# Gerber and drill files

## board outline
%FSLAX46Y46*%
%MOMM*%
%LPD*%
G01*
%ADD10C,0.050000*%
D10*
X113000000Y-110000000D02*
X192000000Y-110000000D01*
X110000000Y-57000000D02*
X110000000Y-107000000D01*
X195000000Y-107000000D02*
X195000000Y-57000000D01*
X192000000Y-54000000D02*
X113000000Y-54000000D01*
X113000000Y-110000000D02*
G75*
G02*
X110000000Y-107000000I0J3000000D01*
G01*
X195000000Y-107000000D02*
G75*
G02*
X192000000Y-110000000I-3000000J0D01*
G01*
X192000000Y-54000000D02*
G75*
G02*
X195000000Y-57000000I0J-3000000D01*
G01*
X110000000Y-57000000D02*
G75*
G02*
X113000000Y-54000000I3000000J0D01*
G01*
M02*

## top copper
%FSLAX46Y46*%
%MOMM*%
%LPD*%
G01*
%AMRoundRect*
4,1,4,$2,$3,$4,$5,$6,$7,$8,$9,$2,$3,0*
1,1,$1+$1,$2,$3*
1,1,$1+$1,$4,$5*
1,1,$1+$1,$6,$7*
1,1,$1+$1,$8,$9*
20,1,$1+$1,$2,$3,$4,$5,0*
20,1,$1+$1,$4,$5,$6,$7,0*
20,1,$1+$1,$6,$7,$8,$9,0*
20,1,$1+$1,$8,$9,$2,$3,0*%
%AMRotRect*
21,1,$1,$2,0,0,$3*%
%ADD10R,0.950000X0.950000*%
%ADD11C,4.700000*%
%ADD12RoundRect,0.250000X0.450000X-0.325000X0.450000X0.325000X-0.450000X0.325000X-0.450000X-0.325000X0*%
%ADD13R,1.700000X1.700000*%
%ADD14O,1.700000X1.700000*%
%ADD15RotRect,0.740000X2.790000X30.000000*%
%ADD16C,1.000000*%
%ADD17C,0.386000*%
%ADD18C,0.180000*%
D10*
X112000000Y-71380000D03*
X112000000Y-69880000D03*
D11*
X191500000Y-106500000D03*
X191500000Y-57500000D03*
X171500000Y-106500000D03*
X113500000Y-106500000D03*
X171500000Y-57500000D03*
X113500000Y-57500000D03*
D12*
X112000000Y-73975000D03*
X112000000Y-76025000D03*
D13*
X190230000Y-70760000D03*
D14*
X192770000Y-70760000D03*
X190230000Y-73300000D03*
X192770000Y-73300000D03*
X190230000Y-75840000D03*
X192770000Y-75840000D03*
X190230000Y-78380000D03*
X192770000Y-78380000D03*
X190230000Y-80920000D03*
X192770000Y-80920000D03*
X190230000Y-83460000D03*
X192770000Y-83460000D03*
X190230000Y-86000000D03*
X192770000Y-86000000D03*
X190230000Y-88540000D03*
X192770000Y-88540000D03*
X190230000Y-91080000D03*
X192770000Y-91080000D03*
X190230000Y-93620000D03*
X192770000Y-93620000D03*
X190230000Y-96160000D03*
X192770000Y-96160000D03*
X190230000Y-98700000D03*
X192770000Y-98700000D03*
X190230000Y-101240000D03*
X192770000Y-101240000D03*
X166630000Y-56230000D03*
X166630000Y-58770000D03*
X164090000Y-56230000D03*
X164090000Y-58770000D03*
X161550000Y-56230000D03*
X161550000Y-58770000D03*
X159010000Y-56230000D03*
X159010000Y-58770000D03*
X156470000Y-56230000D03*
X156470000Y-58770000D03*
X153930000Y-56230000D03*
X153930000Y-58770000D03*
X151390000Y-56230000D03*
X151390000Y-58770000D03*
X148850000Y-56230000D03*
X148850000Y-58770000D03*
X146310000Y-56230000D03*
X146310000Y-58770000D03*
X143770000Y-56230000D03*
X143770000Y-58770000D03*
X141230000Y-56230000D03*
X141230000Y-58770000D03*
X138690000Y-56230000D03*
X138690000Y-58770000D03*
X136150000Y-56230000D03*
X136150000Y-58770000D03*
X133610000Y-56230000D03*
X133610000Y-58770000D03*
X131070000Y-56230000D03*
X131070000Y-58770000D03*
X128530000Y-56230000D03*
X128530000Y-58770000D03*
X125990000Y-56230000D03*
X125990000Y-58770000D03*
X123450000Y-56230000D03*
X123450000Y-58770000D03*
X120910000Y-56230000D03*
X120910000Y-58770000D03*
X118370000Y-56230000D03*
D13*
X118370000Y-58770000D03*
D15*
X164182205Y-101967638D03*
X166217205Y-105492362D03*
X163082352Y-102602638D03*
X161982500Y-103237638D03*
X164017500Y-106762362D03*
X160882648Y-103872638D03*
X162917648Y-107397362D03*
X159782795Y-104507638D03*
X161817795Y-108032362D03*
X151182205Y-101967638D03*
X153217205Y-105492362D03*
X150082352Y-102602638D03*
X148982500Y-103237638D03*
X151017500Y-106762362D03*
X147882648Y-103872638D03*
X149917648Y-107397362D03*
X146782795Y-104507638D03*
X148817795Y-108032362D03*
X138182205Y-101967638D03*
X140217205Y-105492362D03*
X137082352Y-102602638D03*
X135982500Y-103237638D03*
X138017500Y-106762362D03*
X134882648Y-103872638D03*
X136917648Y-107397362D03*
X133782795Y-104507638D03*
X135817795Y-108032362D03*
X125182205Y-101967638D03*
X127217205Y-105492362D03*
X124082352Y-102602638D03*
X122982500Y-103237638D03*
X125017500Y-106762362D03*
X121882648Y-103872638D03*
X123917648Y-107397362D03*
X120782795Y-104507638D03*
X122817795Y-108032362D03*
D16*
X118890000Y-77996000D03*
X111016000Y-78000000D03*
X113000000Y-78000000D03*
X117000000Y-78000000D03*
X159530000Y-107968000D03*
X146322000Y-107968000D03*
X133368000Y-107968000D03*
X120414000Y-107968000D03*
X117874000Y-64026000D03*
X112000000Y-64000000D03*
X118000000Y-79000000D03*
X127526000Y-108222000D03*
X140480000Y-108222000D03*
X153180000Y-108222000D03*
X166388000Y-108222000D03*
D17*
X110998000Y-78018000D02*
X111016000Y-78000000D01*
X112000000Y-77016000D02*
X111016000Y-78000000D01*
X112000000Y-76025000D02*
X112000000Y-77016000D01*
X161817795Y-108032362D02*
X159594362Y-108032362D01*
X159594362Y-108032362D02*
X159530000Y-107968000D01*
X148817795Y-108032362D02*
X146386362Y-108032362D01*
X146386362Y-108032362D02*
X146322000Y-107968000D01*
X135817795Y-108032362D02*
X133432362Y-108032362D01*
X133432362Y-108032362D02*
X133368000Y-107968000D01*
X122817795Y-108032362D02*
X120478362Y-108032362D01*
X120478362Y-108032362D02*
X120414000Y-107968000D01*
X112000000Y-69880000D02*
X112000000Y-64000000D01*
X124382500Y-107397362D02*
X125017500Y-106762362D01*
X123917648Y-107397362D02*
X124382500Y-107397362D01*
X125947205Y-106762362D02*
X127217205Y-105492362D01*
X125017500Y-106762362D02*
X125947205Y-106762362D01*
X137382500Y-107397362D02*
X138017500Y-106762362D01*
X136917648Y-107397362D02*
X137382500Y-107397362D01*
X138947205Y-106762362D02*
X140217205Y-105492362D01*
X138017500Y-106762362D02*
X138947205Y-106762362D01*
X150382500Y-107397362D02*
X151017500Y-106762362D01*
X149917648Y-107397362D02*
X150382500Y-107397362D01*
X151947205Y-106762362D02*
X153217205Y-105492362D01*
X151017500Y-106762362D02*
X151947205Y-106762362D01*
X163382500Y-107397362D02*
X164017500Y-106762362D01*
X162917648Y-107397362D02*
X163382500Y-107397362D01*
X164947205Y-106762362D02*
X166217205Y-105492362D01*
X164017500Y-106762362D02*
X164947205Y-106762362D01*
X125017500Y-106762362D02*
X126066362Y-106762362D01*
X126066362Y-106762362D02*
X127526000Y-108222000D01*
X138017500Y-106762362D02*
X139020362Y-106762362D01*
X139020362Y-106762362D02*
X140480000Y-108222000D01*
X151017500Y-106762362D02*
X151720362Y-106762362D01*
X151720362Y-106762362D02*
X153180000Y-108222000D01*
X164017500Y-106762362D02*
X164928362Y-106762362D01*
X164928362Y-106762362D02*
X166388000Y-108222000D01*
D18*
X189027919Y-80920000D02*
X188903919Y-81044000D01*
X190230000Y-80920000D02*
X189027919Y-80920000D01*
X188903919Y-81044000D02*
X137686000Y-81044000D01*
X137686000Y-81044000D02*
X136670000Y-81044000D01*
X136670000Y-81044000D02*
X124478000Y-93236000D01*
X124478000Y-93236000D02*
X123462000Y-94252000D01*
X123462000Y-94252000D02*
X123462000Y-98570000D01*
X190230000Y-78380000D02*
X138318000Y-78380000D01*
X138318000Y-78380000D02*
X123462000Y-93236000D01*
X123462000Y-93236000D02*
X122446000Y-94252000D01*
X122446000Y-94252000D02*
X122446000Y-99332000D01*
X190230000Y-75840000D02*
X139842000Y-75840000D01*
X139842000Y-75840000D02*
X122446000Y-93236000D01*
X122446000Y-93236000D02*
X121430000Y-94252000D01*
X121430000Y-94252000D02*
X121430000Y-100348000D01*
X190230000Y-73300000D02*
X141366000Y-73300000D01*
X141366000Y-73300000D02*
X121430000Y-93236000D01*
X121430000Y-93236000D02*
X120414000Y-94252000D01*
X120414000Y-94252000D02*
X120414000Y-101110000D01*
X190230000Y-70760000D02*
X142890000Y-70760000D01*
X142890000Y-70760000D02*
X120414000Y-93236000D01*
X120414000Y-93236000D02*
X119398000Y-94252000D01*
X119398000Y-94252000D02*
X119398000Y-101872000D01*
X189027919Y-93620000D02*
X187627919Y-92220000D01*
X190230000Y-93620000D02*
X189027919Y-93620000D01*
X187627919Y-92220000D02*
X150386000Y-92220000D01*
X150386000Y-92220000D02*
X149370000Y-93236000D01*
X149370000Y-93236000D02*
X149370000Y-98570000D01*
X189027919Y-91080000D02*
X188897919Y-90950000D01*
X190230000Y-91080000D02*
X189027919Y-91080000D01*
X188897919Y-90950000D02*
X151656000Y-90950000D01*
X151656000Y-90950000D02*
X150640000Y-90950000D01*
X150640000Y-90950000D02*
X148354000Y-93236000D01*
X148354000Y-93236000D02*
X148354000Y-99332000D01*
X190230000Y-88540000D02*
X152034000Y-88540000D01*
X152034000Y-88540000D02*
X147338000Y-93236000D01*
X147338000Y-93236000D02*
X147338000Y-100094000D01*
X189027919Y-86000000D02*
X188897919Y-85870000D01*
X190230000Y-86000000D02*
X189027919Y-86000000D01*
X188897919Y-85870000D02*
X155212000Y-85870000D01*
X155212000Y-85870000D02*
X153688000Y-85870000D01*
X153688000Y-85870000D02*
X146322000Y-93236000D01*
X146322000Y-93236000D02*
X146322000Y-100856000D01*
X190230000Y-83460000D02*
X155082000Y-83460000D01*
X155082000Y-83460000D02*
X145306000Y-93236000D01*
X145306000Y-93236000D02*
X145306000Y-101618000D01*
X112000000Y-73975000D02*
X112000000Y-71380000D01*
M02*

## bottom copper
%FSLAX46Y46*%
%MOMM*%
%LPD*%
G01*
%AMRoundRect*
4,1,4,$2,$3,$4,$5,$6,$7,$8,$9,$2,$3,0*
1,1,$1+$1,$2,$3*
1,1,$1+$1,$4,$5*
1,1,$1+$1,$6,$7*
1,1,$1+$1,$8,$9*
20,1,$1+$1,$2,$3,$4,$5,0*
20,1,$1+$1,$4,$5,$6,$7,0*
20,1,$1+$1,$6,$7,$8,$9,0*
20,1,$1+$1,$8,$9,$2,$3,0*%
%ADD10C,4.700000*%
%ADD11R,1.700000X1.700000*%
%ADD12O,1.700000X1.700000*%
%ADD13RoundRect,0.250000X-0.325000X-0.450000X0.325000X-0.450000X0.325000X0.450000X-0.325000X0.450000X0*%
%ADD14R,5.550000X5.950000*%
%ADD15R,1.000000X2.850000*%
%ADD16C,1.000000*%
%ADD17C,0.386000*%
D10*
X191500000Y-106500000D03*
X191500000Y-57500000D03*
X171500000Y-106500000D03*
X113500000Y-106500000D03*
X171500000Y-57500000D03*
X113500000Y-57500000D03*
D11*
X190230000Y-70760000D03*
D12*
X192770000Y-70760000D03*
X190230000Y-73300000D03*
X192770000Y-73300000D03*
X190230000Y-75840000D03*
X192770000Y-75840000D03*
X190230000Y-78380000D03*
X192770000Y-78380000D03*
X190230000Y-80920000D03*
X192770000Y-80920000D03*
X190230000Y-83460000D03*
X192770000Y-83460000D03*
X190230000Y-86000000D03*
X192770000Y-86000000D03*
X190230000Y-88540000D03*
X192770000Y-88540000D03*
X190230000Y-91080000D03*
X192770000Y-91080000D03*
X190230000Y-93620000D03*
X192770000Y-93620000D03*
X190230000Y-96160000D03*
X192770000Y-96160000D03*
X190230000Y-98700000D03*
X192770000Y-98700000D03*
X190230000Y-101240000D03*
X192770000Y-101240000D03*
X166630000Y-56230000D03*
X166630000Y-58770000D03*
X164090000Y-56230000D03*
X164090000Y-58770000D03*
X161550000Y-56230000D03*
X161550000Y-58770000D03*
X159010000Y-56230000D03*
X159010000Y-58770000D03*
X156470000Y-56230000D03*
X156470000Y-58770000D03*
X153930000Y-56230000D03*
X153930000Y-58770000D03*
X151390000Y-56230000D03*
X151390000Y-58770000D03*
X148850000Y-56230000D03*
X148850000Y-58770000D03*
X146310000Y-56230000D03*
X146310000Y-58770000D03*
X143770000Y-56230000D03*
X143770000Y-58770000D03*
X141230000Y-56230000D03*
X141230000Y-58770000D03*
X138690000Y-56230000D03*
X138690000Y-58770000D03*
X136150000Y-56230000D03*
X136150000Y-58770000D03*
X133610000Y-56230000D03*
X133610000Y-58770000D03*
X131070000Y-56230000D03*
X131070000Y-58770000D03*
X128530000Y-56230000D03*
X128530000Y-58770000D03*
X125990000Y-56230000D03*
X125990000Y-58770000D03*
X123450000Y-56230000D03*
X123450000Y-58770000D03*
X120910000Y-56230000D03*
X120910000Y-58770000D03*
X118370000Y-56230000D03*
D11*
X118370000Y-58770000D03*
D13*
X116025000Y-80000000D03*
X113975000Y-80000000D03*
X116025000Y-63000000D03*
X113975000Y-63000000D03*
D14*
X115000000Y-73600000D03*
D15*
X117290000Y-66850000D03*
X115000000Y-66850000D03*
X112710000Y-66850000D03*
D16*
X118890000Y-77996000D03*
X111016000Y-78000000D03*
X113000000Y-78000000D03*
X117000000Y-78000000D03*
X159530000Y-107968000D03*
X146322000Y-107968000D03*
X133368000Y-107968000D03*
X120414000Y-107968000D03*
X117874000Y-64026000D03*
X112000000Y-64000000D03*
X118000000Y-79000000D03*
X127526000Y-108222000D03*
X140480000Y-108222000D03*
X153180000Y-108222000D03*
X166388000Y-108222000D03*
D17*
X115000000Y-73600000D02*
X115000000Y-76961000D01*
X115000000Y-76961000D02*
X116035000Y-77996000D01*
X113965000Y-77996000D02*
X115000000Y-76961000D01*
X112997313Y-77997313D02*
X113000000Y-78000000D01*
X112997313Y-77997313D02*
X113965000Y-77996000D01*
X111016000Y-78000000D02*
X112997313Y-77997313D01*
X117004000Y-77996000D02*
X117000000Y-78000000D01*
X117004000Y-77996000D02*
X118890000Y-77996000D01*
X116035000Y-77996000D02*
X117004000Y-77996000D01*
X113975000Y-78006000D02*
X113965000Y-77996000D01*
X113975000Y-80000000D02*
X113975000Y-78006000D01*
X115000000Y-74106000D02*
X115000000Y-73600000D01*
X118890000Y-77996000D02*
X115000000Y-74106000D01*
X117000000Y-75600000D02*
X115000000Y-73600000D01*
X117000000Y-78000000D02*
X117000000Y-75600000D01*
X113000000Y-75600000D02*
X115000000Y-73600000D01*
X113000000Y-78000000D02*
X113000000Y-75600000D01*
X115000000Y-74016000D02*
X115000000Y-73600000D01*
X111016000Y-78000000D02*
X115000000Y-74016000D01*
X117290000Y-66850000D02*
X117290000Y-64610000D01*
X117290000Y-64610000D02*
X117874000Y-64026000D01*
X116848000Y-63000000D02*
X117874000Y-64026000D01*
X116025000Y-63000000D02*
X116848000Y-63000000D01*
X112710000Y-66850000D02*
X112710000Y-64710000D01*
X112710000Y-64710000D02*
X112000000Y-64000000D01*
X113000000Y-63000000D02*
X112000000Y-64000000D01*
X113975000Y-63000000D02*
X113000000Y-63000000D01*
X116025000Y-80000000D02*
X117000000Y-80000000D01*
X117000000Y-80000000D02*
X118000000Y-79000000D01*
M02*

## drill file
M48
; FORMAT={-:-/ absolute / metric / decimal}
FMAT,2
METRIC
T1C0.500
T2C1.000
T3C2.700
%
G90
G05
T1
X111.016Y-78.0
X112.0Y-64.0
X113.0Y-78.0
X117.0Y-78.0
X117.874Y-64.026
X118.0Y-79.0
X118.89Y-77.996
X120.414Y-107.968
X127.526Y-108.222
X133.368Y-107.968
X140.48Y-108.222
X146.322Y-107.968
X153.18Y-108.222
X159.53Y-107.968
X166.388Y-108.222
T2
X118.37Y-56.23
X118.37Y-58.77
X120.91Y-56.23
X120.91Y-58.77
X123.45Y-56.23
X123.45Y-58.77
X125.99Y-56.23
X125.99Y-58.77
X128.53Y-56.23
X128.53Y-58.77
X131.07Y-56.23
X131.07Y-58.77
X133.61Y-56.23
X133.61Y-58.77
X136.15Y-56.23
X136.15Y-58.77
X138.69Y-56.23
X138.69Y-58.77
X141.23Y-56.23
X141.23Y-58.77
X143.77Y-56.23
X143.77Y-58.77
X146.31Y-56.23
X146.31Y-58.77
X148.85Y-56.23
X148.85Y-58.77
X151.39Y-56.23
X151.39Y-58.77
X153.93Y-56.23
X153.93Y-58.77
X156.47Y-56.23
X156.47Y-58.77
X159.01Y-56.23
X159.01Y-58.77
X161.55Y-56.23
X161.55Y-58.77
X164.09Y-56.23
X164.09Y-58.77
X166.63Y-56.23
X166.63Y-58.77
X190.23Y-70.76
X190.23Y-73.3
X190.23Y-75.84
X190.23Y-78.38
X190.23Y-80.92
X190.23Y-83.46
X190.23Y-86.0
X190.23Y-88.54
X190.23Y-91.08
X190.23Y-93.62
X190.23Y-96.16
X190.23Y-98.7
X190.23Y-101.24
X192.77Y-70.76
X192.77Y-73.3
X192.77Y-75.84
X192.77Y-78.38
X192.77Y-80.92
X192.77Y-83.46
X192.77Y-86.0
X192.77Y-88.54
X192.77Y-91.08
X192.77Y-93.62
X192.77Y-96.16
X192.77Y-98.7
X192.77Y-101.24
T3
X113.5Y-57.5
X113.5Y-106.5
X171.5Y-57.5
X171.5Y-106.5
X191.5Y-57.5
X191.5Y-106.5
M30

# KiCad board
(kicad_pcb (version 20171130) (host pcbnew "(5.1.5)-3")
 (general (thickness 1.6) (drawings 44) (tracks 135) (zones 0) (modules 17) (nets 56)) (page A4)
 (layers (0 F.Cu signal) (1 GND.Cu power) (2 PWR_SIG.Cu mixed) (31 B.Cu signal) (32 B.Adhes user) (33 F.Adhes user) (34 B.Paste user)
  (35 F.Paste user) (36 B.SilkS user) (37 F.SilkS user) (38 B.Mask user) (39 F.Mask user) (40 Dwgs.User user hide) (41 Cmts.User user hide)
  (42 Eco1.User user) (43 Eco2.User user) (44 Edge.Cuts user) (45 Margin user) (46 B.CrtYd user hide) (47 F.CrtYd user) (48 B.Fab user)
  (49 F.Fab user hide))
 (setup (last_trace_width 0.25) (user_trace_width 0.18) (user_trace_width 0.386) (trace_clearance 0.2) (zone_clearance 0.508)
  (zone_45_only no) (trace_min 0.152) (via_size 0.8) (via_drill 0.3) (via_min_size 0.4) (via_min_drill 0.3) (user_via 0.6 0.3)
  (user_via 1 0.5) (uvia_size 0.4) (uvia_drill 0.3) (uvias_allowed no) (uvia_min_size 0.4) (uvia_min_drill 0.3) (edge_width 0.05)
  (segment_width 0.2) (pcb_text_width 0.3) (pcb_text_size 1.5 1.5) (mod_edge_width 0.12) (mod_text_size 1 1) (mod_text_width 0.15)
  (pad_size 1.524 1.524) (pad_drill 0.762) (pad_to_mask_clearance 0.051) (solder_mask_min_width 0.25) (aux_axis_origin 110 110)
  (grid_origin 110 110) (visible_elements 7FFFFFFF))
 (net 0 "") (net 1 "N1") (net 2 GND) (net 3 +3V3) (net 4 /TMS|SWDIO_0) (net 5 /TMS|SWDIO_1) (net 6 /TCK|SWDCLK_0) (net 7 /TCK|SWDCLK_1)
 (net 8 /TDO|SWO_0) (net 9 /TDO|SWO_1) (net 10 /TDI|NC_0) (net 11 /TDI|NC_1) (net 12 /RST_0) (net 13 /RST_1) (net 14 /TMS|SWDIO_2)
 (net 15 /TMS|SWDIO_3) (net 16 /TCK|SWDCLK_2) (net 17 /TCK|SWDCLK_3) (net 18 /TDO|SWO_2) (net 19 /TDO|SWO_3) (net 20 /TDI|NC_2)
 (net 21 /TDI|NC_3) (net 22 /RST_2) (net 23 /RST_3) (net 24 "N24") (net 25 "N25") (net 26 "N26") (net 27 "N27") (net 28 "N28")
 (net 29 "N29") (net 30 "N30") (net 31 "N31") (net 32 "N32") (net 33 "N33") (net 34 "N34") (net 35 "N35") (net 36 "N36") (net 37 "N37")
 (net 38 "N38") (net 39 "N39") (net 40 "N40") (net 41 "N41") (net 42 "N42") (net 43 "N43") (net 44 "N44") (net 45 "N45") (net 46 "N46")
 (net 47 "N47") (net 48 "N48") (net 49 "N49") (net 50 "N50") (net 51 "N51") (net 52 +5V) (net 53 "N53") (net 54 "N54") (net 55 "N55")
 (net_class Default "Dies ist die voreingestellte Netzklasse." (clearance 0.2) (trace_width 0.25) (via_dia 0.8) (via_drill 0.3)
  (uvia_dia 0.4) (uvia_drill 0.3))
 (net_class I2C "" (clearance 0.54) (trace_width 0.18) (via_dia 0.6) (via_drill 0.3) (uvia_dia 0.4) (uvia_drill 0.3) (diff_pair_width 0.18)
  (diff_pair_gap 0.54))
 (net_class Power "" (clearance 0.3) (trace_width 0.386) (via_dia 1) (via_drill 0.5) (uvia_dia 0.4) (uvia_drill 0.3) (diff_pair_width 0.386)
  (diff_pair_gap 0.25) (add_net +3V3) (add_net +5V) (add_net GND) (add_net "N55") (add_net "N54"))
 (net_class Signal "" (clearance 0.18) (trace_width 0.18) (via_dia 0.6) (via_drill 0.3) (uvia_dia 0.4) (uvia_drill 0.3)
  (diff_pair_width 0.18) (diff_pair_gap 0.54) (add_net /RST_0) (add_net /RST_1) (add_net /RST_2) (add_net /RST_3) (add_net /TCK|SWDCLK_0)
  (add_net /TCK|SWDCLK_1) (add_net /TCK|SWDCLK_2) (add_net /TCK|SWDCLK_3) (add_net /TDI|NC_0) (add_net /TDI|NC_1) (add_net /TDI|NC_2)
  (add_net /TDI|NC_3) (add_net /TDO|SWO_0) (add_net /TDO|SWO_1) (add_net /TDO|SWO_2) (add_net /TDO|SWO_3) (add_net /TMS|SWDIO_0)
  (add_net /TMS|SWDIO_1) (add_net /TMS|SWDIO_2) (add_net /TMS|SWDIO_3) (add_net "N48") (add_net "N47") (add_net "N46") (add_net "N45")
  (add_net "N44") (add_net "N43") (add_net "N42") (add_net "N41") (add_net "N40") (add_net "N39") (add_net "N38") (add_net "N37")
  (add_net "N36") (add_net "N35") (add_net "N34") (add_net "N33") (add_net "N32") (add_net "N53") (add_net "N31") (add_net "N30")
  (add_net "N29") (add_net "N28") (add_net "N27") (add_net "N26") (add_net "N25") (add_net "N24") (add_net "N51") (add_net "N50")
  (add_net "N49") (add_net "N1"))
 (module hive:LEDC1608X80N (layer F.Cu) (at 112 70.63 270)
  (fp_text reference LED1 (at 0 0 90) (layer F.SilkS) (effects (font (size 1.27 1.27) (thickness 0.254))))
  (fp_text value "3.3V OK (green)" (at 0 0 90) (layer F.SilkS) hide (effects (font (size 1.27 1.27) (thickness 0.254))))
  (pad 2 smd rect (at 0.75 0) (size 0.95 0.95) (layers F.Cu F.Paste F.Mask) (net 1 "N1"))
  (pad 1 smd rect (at -0.75 0) (size 0.95 0.95) (layers F.Cu F.Paste F.Mask) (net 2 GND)))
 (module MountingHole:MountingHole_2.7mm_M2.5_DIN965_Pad (layer F.Cu) (at 191.5 106.5)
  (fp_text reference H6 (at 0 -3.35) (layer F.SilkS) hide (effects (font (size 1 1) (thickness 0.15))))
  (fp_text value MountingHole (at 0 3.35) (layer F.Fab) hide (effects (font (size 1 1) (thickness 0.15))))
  (pad 1 thru_hole circle (at 0 0) (size 4.7 4.7) (drill 2.7) (layers *.Cu *.Mask) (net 2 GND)))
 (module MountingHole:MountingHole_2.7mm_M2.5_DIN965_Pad (layer F.Cu) (at 191.5 57.5)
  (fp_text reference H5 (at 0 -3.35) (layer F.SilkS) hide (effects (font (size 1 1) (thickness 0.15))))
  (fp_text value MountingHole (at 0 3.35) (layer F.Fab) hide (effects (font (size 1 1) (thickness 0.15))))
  (pad 1 thru_hole circle (at 0 0) (size 4.7 4.7) (drill 2.7) (layers *.Cu *.Mask) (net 2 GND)))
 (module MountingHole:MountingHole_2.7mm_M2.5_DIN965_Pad (layer F.Cu) (at 171.5 106.5)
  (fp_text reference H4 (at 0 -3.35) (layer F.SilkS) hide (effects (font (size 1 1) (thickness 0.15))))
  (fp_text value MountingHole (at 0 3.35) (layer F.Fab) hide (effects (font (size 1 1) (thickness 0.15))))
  (pad 1 thru_hole circle (at 0 0) (size 4.7 4.7) (drill 2.7) (layers *.Cu *.Mask) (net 2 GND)))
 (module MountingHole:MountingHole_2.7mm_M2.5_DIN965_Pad (layer F.Cu) (at 113.5 106.5)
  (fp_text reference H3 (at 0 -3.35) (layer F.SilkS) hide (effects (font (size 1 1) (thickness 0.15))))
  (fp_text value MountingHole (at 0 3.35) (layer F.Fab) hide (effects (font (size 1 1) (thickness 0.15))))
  (pad 1 thru_hole circle (at 0 0) (size 4.7 4.7) (drill 2.7) (layers *.Cu *.Mask) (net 2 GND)))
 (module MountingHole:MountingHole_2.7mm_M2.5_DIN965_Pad (layer F.Cu) (at 171.5 57.5)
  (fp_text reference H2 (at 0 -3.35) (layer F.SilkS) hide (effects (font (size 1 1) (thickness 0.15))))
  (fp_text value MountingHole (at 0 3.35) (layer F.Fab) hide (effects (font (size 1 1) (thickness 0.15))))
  (pad 1 thru_hole circle (at 0 0) (size 4.7 4.7) (drill 2.7) (layers *.Cu *.Mask) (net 2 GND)))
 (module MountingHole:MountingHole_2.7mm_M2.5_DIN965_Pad (layer F.Cu) (at 113.5 57.5)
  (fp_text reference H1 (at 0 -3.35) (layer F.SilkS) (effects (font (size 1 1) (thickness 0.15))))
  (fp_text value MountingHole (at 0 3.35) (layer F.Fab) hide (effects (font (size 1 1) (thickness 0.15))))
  (pad 1 thru_hole circle (at 0 0) (size 4.7 4.7) (drill 2.7) (layers *.Cu *.Mask) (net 2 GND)))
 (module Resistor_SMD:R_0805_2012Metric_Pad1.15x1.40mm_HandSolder (layer F.Cu) (at 112 75 90)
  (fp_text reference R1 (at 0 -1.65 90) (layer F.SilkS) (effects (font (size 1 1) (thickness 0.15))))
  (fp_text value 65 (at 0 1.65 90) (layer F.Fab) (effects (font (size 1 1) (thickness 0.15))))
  (pad 2 smd roundrect (at 1.025 0 90) (size 1.15 1.4) (layers F.Cu F.Paste F.Mask) (roundrect_rratio 0.217391) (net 1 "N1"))
  (pad 1 smd roundrect (at -1.025 0 90) (size 1.15 1.4) (layers F.Cu F.Paste F.Mask) (roundrect_rratio 0.217391) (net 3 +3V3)))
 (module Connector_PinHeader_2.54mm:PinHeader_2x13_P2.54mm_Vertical (layer F.Cu) (at 190.23 70.76)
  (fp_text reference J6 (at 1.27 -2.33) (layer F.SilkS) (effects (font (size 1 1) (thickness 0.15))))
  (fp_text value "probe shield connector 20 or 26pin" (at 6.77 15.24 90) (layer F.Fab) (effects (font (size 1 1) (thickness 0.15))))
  (pad 1 thru_hole rect (at 0 0) (size 1.7 1.7) (drill 1) (layers *.Cu *.Mask) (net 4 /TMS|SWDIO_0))
  (pad 2 thru_hole oval (at 2.54 0) (size 1.7 1.7) (drill 1) (layers *.Cu *.Mask) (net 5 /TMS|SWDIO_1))
  (pad 3 thru_hole oval (at 0 2.54) (size 1.7 1.7) (drill 1) (layers *.Cu *.Mask) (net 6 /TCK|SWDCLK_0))
  (pad 4 thru_hole oval (at 2.54 2.54) (size 1.7 1.7) (drill 1) (layers *.Cu *.Mask) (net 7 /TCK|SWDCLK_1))
  (pad 5 thru_hole oval (at 0 5.08) (size 1.7 1.7) (drill 1) (layers *.Cu *.Mask) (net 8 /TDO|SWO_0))
  (pad 6 thru_hole oval (at 2.54 5.08) (size 1.7 1.7) (drill 1) (layers *.Cu *.Mask) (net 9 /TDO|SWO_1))
  (pad 7 thru_hole oval (at 0 7.62) (size 1.7 1.7) (drill 1) (layers *.Cu *.Mask) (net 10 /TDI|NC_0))
  (pad 8 thru_hole oval (at 2.54 7.62) (size 1.7 1.7) (drill 1) (layers *.Cu *.Mask) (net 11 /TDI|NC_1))
  (pad 9 thru_hole oval (at 0 10.16) (size 1.7 1.7) (drill 1) (layers *.Cu *.Mask) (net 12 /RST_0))
  (pad 10 thru_hole oval (at 2.54 10.16) (size 1.7 1.7) (drill 1) (layers *.Cu *.Mask) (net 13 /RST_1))
  (pad 11 thru_hole oval (at 0 12.7) (size 1.7 1.7) (drill 1) (layers *.Cu *.Mask) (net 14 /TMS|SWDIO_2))
  (pad 12 thru_hole oval (at 2.54 12.7) (size 1.7 1.7) (drill 1) (layers *.Cu *.Mask) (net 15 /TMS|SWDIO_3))
  (pad 13 thru_hole oval (at 0 15.24) (size 1.7 1.7) (drill 1) (layers *.Cu *.Mask) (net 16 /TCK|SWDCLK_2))
  (pad 14 thru_hole oval (at 2.54 15.24) (size 1.7 1.7) (drill 1) (layers *.Cu *.Mask) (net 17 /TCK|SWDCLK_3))
  (pad 15 thru_hole oval (at 0 17.78) (size 1.7 1.7) (drill 1) (layers *.Cu *.Mask) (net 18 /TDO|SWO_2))
  (pad 16 thru_hole oval (at 2.54 17.78) (size 1.7 1.7) (drill 1) (layers *.Cu *.Mask) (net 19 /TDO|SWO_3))
  (pad 17 thru_hole oval (at 0 20.32) (size 1.7 1.7) (drill 1) (layers *.Cu *.Mask) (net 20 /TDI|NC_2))
  (pad 18 thru_hole oval (at 2.54 20.32) (size 1.7 1.7) (drill 1) (layers *.Cu *.Mask) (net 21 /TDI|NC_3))
  (pad 19 thru_hole oval (at 0 22.86) (size 1.7 1.7) (drill 1) (layers *.Cu *.Mask) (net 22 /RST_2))
  (pad 20 thru_hole oval (at 2.54 22.86) (size 1.7 1.7) (drill 1) (layers *.Cu *.Mask) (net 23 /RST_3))
  (pad 21 thru_hole oval (at 0 25.4) (size 1.7 1.7) (drill 1) (layers *.Cu *.Mask) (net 2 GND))
  (pad 22 thru_hole oval (at 2.54 25.4) (size 1.7 1.7) (drill 1) (layers *.Cu *.Mask) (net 2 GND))
  (pad 23 thru_hole oval (at 0 27.94) (size 1.7 1.7) (drill 1) (layers *.Cu *.Mask) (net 2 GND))
  (pad 24 thru_hole oval (at 2.54 27.94) (size 1.7 1.7) (drill 1) (layers *.Cu *.Mask) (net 2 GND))
  (pad 25 thru_hole oval (at 0 30.48) (size 1.7 1.7) (drill 1) (layers *.Cu *.Mask) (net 2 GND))
  (pad 26 thru_hole oval (at 2.54 30.48) (size 1.7 1.7) (drill 1) (layers *.Cu *.Mask) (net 2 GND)))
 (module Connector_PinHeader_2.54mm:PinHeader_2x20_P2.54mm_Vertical (layer F.Cu) (at 118.37 58.77 90)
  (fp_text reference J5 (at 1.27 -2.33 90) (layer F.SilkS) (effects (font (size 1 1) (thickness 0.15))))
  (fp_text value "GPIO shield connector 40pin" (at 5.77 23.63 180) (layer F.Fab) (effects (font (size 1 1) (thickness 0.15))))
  (pad 40 thru_hole oval (at 2.54 48.26 90) (size 1.7 1.7) (drill 1) (layers *.Cu *.Mask) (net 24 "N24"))
  (pad 39 thru_hole oval (at 0 48.26 90) (size 1.7 1.7) (drill 1) (layers *.Cu *.Mask) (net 2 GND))
  (pad 38 thru_hole oval (at 2.54 45.72 90) (size 1.7 1.7) (drill 1) (layers *.Cu *.Mask) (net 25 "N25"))
  (pad 37 thru_hole oval (at 0 45.72 90) (size 1.7 1.7) (drill 1) (layers *.Cu *.Mask) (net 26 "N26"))
  (pad 36 thru_hole oval (at 2.54 43.18 90) (size 1.7 1.7) (drill 1) (layers *.Cu *.Mask) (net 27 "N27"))
  (pad 35 thru_hole oval (at 0 43.18 90) (size 1.7 1.7) (drill 1) (layers *.Cu *.Mask) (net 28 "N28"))
  (pad 34 thru_hole oval (at 2.54 40.64 90) (size 1.7 1.7) (drill 1) (layers *.Cu *.Mask) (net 2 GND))
  (pad 33 thru_hole oval (at 0 40.64 90) (size 1.7 1.7) (drill 1) (layers *.Cu *.Mask) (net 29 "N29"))
  (pad 32 thru_hole oval (at 2.54 38.1 90) (size 1.7 1.7) (drill 1) (layers *.Cu *.Mask) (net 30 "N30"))
  (pad 31 thru_hole oval (at 0 38.1 90) (size 1.7 1.7) (drill 1) (layers *.Cu *.Mask) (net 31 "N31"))
  (pad 30 thru_hole oval (at 2.54 35.56 90) (size 1.7 1.7) (drill 1) (layers *.Cu *.Mask) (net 2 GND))
  (pad 29 thru_hole oval (at 0 35.56 90) (size 1.7 1.7) (drill 1) (layers *.Cu *.Mask) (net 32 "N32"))
  (pad 28 thru_hole oval (at 2.54 33.02 90) (size 1.7 1.7) (drill 1) (layers *.Cu *.Mask) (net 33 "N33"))
  (pad 27 thru_hole oval (at 0 33.02 90) (size 1.7 1.7) (drill 1) (layers *.Cu *.Mask) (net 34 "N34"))
  (pad 26 thru_hole oval (at 2.54 30.48 90) (size 1.7 1.7) (drill 1) (layers *.Cu *.Mask) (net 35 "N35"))
  (pad 25 thru_hole oval (at 0 30.48 90) (size 1.7 1.7) (drill 1) (layers *.Cu *.Mask) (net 2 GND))
  (pad 24 thru_hole oval (at 2.54 27.94 90) (size 1.7 1.7) (drill 1) (layers *.Cu *.Mask) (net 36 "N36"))
  (pad 23 thru_hole oval (at 0 27.94 90) (size 1.7 1.7) (drill 1) (layers *.Cu *.Mask) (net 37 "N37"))
  (pad 22 thru_hole oval (at 2.54 25.4 90) (size 1.7 1.7) (drill 1) (layers *.Cu *.Mask) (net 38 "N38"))
  (pad 21 thru_hole oval (at 0 25.4 90) (size 1.7 1.7) (drill 1) (layers *.Cu *.Mask) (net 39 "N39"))
  (pad 20 thru_hole oval (at 2.54 22.86 90) (size 1.7 1.7) (drill 1) (layers *.Cu *.Mask) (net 2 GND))
  (pad 19 thru_hole oval (at 0 22.86 90) (size 1.7 1.7) (drill 1) (layers *.Cu *.Mask) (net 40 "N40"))
  (pad 18 thru_hole oval (at 2.54 20.32 90) (size 1.7 1.7) (drill 1) (layers *.Cu *.Mask) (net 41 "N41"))
  (pad 17 thru_hole oval (at 0 20.32 90) (size 1.7 1.7) (drill 1) (layers *.Cu *.Mask) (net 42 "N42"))
  (pad 16 thru_hole oval (at 2.54 17.78 90) (size 1.7 1.7) (drill 1) (layers *.Cu *.Mask) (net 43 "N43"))
  (pad 15 thru_hole oval (at 0 17.78 90) (size 1.7 1.7) (drill 1) (layers *.Cu *.Mask) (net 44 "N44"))
  (pad 14 thru_hole oval (at 2.54 15.24 90) (size 1.7 1.7) (drill 1) (layers *.Cu *.Mask) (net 2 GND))
  (pad 13 thru_hole oval (at 0 15.24 90) (size 1.7 1.7) (drill 1) (layers *.Cu *.Mask) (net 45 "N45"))
  (pad 12 thru_hole oval (at 2.54 12.7 90) (size 1.7 1.7) (drill 1) (layers *.Cu *.Mask) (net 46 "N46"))
  (pad 11 thru_hole oval (at 0 12.7 90) (size 1.7 1.7) (drill 1) (layers *.Cu *.Mask) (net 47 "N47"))
  (pad 10 thru_hole oval (at 2.54 10.16 90) (size 1.7 1.7) (drill 1) (layers *.Cu *.Mask) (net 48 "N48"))
  (pad 9 thru_hole oval (at 0 10.16 90) (size 1.7 1.7) (drill 1) (layers *.Cu *.Mask) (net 2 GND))
  (pad 8 thru_hole oval (at 2.54 7.62 90) (size 1.7 1.7) (drill 1) (layers *.Cu *.Mask) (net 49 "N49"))
  (pad 7 thru_hole oval (at 0 7.62 90) (size 1.7 1.7) (drill 1) (layers *.Cu *.Mask) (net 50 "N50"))
  (pad 6 thru_hole oval (at 2.54 5.08 90) (size 1.7 1.7) (drill 1) (layers *.Cu *.Mask) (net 2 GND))
  (pad 5 thru_hole oval (at 0 5.08 90) (size 1.7 1.7) (drill 1) (layers *.Cu *.Mask) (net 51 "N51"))
  (pad 4 thru_hole oval (at 2.54 2.54 90) (size 1.7 1.7) (drill 1) (layers *.Cu *.Mask) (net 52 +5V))
  (pad 3 thru_hole oval (at 0 2.54 90) (size 1.7 1.7) (drill 1) (layers *.Cu *.Mask) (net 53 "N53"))
  (pad 2 thru_hole oval (at 2.54 0 90) (size 1.7 1.7) (drill 1) (layers *.Cu *.Mask) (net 52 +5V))
  (pad 1 thru_hole rect (at 0 0 90) (size 1.7 1.7) (drill 1) (layers *.Cu *.Mask) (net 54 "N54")))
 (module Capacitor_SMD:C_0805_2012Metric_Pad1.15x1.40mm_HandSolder (layer B.Cu) (at 115 80)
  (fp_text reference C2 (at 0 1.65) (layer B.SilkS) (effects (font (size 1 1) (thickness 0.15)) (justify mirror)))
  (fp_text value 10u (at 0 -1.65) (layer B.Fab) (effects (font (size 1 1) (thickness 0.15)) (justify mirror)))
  (pad 2 smd roundrect (at 1.025 0) (size 1.15 1.4) (layers B.Cu B.Paste B.Mask) (roundrect_rratio 0.217391) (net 2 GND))
  (pad 1 smd roundrect (at -1.025 0) (size 1.15 1.4) (layers B.Cu B.Paste B.Mask) (roundrect_rratio 0.217391) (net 3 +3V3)))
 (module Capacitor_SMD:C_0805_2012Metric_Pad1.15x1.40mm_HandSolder (layer B.Cu) (at 115 63)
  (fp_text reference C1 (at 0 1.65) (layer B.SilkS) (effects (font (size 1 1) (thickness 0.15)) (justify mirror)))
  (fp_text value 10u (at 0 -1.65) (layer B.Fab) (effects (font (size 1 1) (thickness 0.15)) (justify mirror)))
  (pad 2 smd roundrect (at 1.025 0) (size 1.15 1.4) (layers B.Cu B.Paste B.Mask) (roundrect_rratio 0.217391) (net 52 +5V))
  (pad 1 smd roundrect (at -1.025 0) (size 1.15 1.4) (layers B.Cu B.Paste B.Mask) (roundrect_rratio 0.217391) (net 2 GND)))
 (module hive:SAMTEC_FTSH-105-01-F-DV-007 (layer F.Cu) (at 163 105 30)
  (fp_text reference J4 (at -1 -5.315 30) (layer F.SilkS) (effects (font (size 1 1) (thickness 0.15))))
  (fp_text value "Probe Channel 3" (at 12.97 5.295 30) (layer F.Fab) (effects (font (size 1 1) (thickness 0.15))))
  (pad 10 smd rect (at 2.54 -2.035 30) (size 0.74 2.79) (layers F.Cu F.Paste F.Mask) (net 23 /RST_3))
  (pad 09 smd rect (at 2.54 2.035 30) (size 0.74 2.79) (layers F.Cu F.Paste F.Mask) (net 2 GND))
  (pad 08 smd rect (at 1.27 -2.035 30) (size 0.74 2.79) (layers F.Cu F.Paste F.Mask) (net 21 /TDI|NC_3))
  (pad 06 smd rect (at 0 -2.035 30) (size 0.74 2.79) (layers F.Cu F.Paste F.Mask) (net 19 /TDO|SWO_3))
  (pad 05 smd rect (at 0 2.035 30) (size 0.74 2.79) (layers F.Cu F.Paste F.Mask) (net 2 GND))
  (pad 04 smd rect (at -1.27 -2.035 30) (size 0.74 2.79) (layers F.Cu F.Paste F.Mask) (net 17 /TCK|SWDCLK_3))
  (pad 03 smd rect (at -1.27 2.035 30) (size 0.74 2.79) (layers F.Cu F.Paste F.Mask) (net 2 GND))
  (pad 02 smd rect (at -2.54 -2.035 30) (size 0.74 2.79) (layers F.Cu F.Paste F.Mask) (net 15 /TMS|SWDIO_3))
  (pad 01 smd rect (at -2.54 2.035 30) (size 0.74 2.79) (layers F.Cu F.Paste F.Mask) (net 3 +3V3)))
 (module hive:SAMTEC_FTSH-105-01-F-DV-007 (layer F.Cu) (at 150 105 30)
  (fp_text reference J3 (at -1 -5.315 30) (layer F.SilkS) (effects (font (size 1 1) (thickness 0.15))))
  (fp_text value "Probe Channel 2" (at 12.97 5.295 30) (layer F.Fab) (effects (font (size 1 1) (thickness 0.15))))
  (pad 10 smd rect (at 2.54 -2.035 30) (size 0.74 2.79) (layers F.Cu F.Paste F.Mask) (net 22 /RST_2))
  (pad 09 smd rect (at 2.54 2.035 30) (size 0.74 2.79) (layers F.Cu F.Paste F.Mask) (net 2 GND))
  (pad 08 smd rect (at 1.27 -2.035 30) (size 0.74 2.79) (layers F.Cu F.Paste F.Mask) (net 20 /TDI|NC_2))
  (pad 06 smd rect (at 0 -2.035 30) (size 0.74 2.79) (layers F.Cu F.Paste F.Mask) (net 18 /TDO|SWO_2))
  (pad 05 smd rect (at 0 2.035 30) (size 0.74 2.79) (layers F.Cu F.Paste F.Mask) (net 2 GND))
  (pad 04 smd rect (at -1.27 -2.035 30) (size 0.74 2.79) (layers F.Cu F.Paste F.Mask) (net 16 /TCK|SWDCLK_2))
  (pad 03 smd rect (at -1.27 2.035 30) (size 0.74 2.79) (layers F.Cu F.Paste F.Mask) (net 2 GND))
  (pad 02 smd rect (at -2.54 -2.035 30) (size 0.74 2.79) (layers F.Cu F.Paste F.Mask) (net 14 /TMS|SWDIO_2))
  (pad 01 smd rect (at -2.54 2.035 30) (size 0.74 2.79) (layers F.Cu F.Paste F.Mask) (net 3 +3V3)))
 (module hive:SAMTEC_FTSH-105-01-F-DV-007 (layer F.Cu) (at 137 105 30)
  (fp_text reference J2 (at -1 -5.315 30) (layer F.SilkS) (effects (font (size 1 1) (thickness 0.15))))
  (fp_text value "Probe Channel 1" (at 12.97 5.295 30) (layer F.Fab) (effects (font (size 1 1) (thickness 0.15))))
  (pad 10 smd rect (at 2.54 -2.035 30) (size 0.74 2.79) (layers F.Cu F.Paste F.Mask) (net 13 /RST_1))
  (pad 09 smd rect (at 2.54 2.035 30) (size 0.74 2.79) (layers F.Cu F.Paste F.Mask) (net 2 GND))
  (pad 08 smd rect (at 1.27 -2.035 30) (size 0.74 2.79) (layers F.Cu F.Paste F.Mask) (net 11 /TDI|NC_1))
  (pad 06 smd rect (at 0 -2.035 30) (size 0.74 2.79) (layers F.Cu F.Paste F.Mask) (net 9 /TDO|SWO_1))
  (pad 05 smd rect (at 0 2.035 30) (size 0.74 2.79) (layers F.Cu F.Paste F.Mask) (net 2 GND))
  (pad 04 smd rect (at -1.27 -2.035 30) (size 0.74 2.79) (layers F.Cu F.Paste F.Mask) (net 7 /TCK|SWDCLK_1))
  (pad 03 smd rect (at -1.27 2.035 30) (size 0.74 2.79) (layers F.Cu F.Paste F.Mask) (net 2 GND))
  (pad 02 smd rect (at -2.54 -2.035 30) (size 0.74 2.79) (layers F.Cu F.Paste F.Mask) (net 5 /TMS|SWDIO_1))
  (pad 01 smd rect (at -2.54 2.035 30) (size 0.74 2.79) (layers F.Cu F.Paste F.Mask) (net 3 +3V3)))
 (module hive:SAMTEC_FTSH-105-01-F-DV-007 (layer F.Cu) (at 124 105 30)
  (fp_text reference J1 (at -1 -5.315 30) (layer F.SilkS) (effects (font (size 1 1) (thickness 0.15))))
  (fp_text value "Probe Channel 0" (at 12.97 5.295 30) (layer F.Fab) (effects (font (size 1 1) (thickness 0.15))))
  (pad 10 smd rect (at 2.54 -2.035 30) (size 0.74 2.79) (layers F.Cu F.Paste F.Mask) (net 12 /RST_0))
  (pad 09 smd rect (at 2.54 2.035 30) (size 0.74 2.79) (layers F.Cu F.Paste F.Mask) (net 2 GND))
  (pad 08 smd rect (at 1.27 -2.035 30) (size 0.74 2.79) (layers F.Cu F.Paste F.Mask) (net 10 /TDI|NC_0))
  (pad 06 smd rect (at 0 -2.035 30) (size 0.74 2.79) (layers F.Cu F.Paste F.Mask) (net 8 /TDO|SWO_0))
  (pad 05 smd rect (at 0 2.035 30) (size 0.74 2.79) (layers F.Cu F.Paste F.Mask) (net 2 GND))
  (pad 04 smd rect (at -1.27 -2.035 30) (size 0.74 2.79) (layers F.Cu F.Paste F.Mask) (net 6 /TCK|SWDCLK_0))
  (pad 03 smd rect (at -1.27 2.035 30) (size 0.74 2.79) (layers F.Cu F.Paste F.Mask) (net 2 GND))
  (pad 02 smd rect (at -2.54 -2.035 30) (size 0.74 2.79) (layers F.Cu F.Paste F.Mask) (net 4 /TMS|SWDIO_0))
  (pad 01 smd rect (at -2.54 2.035 30) (size 0.74 2.79) (layers F.Cu F.Paste F.Mask) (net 3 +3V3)))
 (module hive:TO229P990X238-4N (layer B.Cu) (at 115 71 270)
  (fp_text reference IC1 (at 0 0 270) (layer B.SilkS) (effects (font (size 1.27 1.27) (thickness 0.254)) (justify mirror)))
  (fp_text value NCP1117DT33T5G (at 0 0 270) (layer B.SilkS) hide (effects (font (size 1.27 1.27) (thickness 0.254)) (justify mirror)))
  (pad 4 smd rect (at 2.6 0 180) (size 5.55 5.95) (layers B.Cu B.Paste B.Mask) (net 3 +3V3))
  (pad 3 smd rect (at -4.15 -2.29 180) (size 1 2.85) (layers B.Cu B.Paste B.Mask) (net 52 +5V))
  (pad 2 smd rect (at -4.15 0 180) (size 1 2.85) (layers B.Cu B.Paste B.Mask) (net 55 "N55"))
  (pad 1 smd rect (at -4.15 2.29 180) (size 1 2.85) (layers B.Cu B.Paste B.Mask) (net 2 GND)))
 (gr_line (start 113 110) (end 192 110) (layer Edge.Cuts) (width 0.05))
 (gr_line (start 110 57) (end 110 107) (layer Edge.Cuts) (width 0.05))
 (gr_line (start 195 107) (end 195 57) (layer Edge.Cuts) (width 0.05))
 (gr_line (start 192 54) (end 113 54) (layer Edge.Cuts) (width 0.05))
 (gr_arc (start 113 107) (end 110 107) (angle -90) (layer Edge.Cuts) (width 0.05))
 (gr_arc (start 192 107) (end 192 110) (angle -90) (layer Edge.Cuts) (width 0.05))
 (gr_arc (start 192 57) (end 195 57) (angle -90) (layer Edge.Cuts) (width 0.05))
 (gr_arc (start 113 57) (end 113 54) (angle -90) (layer Edge.Cuts) (width 0.05))
 (segment (start 115 73.6) (end 115 76.961) (width 0.386) (layer B.Cu) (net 3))
 (via (at 118.89 77.996) (size 1) (drill 0.5) (layers F.Cu B.Cu) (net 3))
 (segment (start 115 76.961) (end 116.035 77.996) (width 0.386) (layer B.Cu) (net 3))
 (segment (start 113.965 77.996) (end 115 76.961) (width 0.386) (layer B.Cu) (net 3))
 (via (at 111.016 78) (size 1) (drill 0.5) (layers F.Cu B.Cu) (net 3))
 (via (at 113 78) (size 1) (drill 0.5) (layers F.Cu B.Cu) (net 3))
 (segment (start 112.997313 77.997313) (end 113 78) (width 0.386) (layer B.Cu) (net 3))
 (segment (start 112.997313 77.997313) (end 113.965 77.996) (width 0.386) (layer B.Cu) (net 3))
 (segment (start 111.016 78) (end 112.997313 77.997313) (width 0.386) (layer B.Cu) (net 3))
 (via (at 117 78) (size 1) (drill 0.5) (layers F.Cu B.Cu) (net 3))
 (segment (start 117.004 77.996) (end 117 78) (width 0.386) (layer B.Cu) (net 3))
 (segment (start 117.004 77.996) (end 118.89 77.996) (width 0.386) (layer B.Cu) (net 3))
 (segment (start 116.035 77.996) (end 117.004 77.996) (width 0.386) (layer B.Cu) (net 3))
 (segment (start 113.975 78.006) (end 113.965 77.996) (width 0.386) (layer B.Cu) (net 3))
 (segment (start 113.975 80) (end 113.975 78.006) (width 0.386) (layer B.Cu) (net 3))
 (segment (start 110.998 78.018) (end 111.016 78) (width 0.386) (layer F.Cu) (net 3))
 (segment (start 112 77.016) (end 111.016 78) (width 0.386) (layer F.Cu) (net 3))
 (segment (start 112 76.025) (end 112 77.016) (width 0.386) (layer F.Cu) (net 3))
 (segment (start 115 74.106) (end 115 73.6) (width 0.386) (layer B.Cu) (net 3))
 (segment (start 118.89 77.996) (end 115 74.106) (width 0.386) (layer B.Cu) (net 3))
 (segment (start 117 75.6) (end 115 73.6) (width 0.386) (layer B.Cu) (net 3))
 (segment (start 117 78) (end 117 75.6) (width 0.386) (layer B.Cu) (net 3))
 (segment (start 113 75.6) (end 115 73.6) (width 0.386) (layer B.Cu) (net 3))
 (segment (start 113 78) (end 113 75.6) (width 0.386) (layer B.Cu) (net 3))
 (segment (start 115 74.016) (end 115 73.6) (width 0.386) (layer B.Cu) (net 3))
 (segment (start 111.016 78) (end 115 74.016) (width 0.386) (layer B.Cu) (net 3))
 (via (at 159.53 107.968) (size 1) (drill 0.5) (layers F.Cu B.Cu) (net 3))
 (segment (start 161.817795 108.032362) (end 159.594362 108.032362) (width 0.386) (layer F.Cu) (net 3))
 (segment (start 159.594362 108.032362) (end 159.53 107.968) (width 0.386) (layer F.Cu) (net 3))
 (via (at 146.322 107.968) (size 1) (drill 0.5) (layers F.Cu B.Cu) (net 3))
 (segment (start 148.817795 108.032362) (end 146.386362 108.032362) (width 0.386) (layer F.Cu) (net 3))
 (segment (start 146.386362 108.032362) (end 146.322 107.968) (width 0.386) (layer F.Cu) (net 3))
 (via (at 133.368 107.968) (size 1) (drill 0.5) (layers F.Cu B.Cu) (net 3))
 (segment (start 135.817795 108.032362) (end 133.432362 108.032362) (width 0.386) (layer F.Cu) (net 3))
 (segment (start 133.432362 108.032362) (end 133.368 107.968) (width 0.386) (layer F.Cu) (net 3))
 (via (at 120.414 107.968) (size 1) (drill 0.5) (layers F.Cu B.Cu) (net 3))
 (segment (start 122.817795 108.032362) (end 120.478362 108.032362) (width 0.386) (layer F.Cu) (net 3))
 (segment (start 120.478362 108.032362) (end 120.414 107.968) (width 0.386) (layer F.Cu) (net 3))
 (segment (start 117.29 66.85) (end 117.29 64.61) (width 0.386) (layer B.Cu) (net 52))
 (via (at 117.874 64.026) (size 1) (drill 0.5) (layers F.Cu B.Cu) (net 52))
 (segment (start 117.29 64.61) (end 117.874 64.026) (width 0.386) (layer B.Cu) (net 52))
 (segment (start 119.669999 57.470001) (end 119.669999 60.452001) (width 0.18) (layer PWR_SIG.Cu) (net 52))
 (segment (start 120.91 56.23) (end 119.669999 57.470001) (width 0.18) (layer PWR_SIG.Cu) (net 52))
 (segment (start 119.610001 57.470001) (end 119.610001 61.190001) (width 0.18) (layer PWR_SIG.Cu) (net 52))
 (segment (start 118.37 56.23) (end 119.610001 57.470001) (width 0.18) (layer PWR_SIG.Cu) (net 52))
 (segment (start 122.192 59.962) (end 122.209999 60.198001) (width 0.18) (layer PWR_SIG.Cu) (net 52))
 (segment (start 122.150001 59.920001) (end 122.192 59.962) (width 0.18) (layer PWR_SIG.Cu) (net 52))
 (segment (start 122.150001 57.470001) (end 122.150001 59.920001) (width 0.18) (layer PWR_SIG.Cu) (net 52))
 (segment (start 120.91 56.23) (end 122.150001 57.470001) (width 0.18) (layer PWR_SIG.Cu) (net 52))
 (segment (start 116.848 63) (end 117.874 64.026) (width 0.386) (layer B.Cu) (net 52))
 (segment (start 116.025 63) (end 116.848 63) (width 0.386) (layer B.Cu) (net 52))
 (segment (start 112.71 66.85) (end 112.71 64.71) (width 0.386) (layer B.Cu) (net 2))
 (via (at 112 64) (size 1) (drill 0.5) (layers F.Cu B.Cu) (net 2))
 (segment (start 112.71 64.71) (end 112 64) (width 0.386) (layer B.Cu) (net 2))
 (segment (start 113 63) (end 112 64) (width 0.386) (layer B.Cu) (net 2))
 (segment (start 113.975 63) (end 113 63) (width 0.386) (layer B.Cu) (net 2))
 (via (at 118 79) (size 1) (drill 0.5) (layers F.Cu B.Cu) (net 2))
 (segment (start 116.025 80) (end 117 80) (width 0.386) (layer B.Cu) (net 2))
 (segment (start 117 80) (end 118 79) (width 0.386) (layer B.Cu) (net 2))
 (segment (start 112 69.88) (end 112 64) (width 0.386) (layer F.Cu) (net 2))
 (segment (start 124.3825 107.397362) (end 125.0175 106.762362) (width 0.386) (layer F.Cu) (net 2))
 (segment (start 123.917648 107.397362) (end 124.3825 107.397362) (width 0.386) (layer F.Cu) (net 2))
 (segment (start 125.947205 106.762362) (end 127.217205 105.492362) (width 0.386) (layer F.Cu) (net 2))
 (segment (start 125.0175 106.762362) (end 125.947205 106.762362) (width 0.386) (layer F.Cu) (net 2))
 (segment (start 137.3825 107.397362) (end 138.0175 106.762362) (width 0.386) (layer F.Cu) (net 2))
 (segment (start 136.917648 107.397362) (end 137.3825 107.397362) (width 0.386) (layer F.Cu) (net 2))
 (segment (start 138.947205 106.762362) (end 140.217205 105.492362) (width 0.386) (layer F.Cu) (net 2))
 (segment (start 138.0175 106.762362) (end 138.947205 106.762362) (width 0.386) (layer F.Cu) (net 2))
 (segment (start 150.3825 107.397362) (end 151.0175 106.762362) (width 0.386) (layer F.Cu) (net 2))
 (segment (start 149.917648 107.397362) (end 150.3825 107.397362) (width 0.386) (layer F.Cu) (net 2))
 (segment (start 151.947205 106.762362) (end 153.217205 105.492362) (width 0.386) (layer F.Cu) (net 2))
 (segment (start 151.0175 106.762362) (end 151.947205 106.762362) (width 0.386) (layer F.Cu) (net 2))
 (segment (start 163.3825 107.397362) (end 164.0175 106.762362) (width 0.386) (layer F.Cu) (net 2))
 (segment (start 162.917648 107.397362) (end 163.3825 107.397362) (width 0.386) (layer F.Cu) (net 2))
 (segment (start 164.947205 106.762362) (end 166.217205 105.492362) (width 0.386) (layer F.Cu) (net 2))
 (segment (start 164.0175 106.762362) (end 164.947205 106.762362) (width 0.386) (layer F.Cu) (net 2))
 (via (at 127.526 108.222) (size 1) (drill 0.5) (layers F.Cu B.Cu) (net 2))
 (segment (start 125.0175 106.762362) (end 126.066362 106.762362) (width 0.386) (layer F.Cu) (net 2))
 (segment (start 126.066362 106.762362) (end 127.526 108.222) (width 0.386) (layer F.Cu) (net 2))
 (via (at 140.48 108.222) (size 1) (drill 0.5) (layers F.Cu B.Cu) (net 2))
 (segment (start 138.0175 106.762362) (end 139.020362 106.762362) (width 0.386) (layer F.Cu) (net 2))
 (segment (start 139.020362 106.762362) (end 140.48 108.222) (width 0.386) (layer F.Cu) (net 2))
 (via (at 153.18 108.222) (size 1) (drill 0.5) (layers F.Cu B.Cu) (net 2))
 (segment (start 151.0175 106.762362) (end 151.720362 106.762362) (width 0.386) (layer F.Cu) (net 2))
 (segment (start 151.720362 106.762362) (end 153.18 108.222) (width 0.386) (layer F.Cu) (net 2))
 (via (at 166.388 108.222) (size 1) (drill 0.5) (layers F.Cu B.Cu) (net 2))
 (segment (start 164.0175 106.762362) (end 164.928362 106.762362) (width 0.386) (layer F.Cu) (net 2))
 (segment (start 164.928362 106.762362) (end 166.388 108.222) (width 0.386) (layer F.Cu) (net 2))
 (segment (start 189.027919 80.92) (end 188.903919 81.044) (width 0.18) (layer F.Cu) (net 12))
 (segment (start 190.23 80.92) (end 189.027919 80.92) (width 0.18) (layer F.Cu) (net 12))
 (segment (start 188.903919 81.044) (end 137.686 81.044) (width 0.18) (layer F.Cu) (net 12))
 (segment (start 137.686 81.044) (end 136.67 81.044) (width 0.18) (layer F.Cu) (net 12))
 (segment (start 136.67 81.044) (end 124.478 93.236) (width 0.18) (layer F.Cu) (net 12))
 (segment (start 124.478 93.236) (end 123.462 94.252) (width 0.18) (layer F.Cu) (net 12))
 (segment (start 123.462 94.252) (end 123.462 98.57) (width 0.18) (layer F.Cu) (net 12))
 (segment (start 190.23 78.38) (end 138.318 78.38) (width 0.18) (layer F.Cu) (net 10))
 (segment (start 138.318 78.38) (end 123.462 93.236) (width 0.18) (layer F.Cu) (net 10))
 (segment (start 123.462 93.236) (end 122.446 94.252) (width 0.18) (layer F.Cu) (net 10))
 (segment (start 122.446 94.252) (end 122.446 99.332) (width 0.18) (layer F.Cu) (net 10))
 (segment (start 190.23 75.84) (end 139.842 75.84) (width 0.18) (layer F.Cu) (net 8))
 (segment (start 139.842 75.84) (end 122.446 93.236) (width 0.18) (layer F.Cu) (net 8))
 (segment (start 122.446 93.236) (end 121.43 94.252) (width 0.18) (layer F.Cu) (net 8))
 (segment (start 121.43 94.252) (end 121.43 100.348) (width 0.18) (layer F.Cu) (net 8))
 (segment (start 190.23 73.3) (end 141.366 73.3) (width 0.18) (layer F.Cu) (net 6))
 (segment (start 141.366 73.3) (end 121.43 93.236) (width 0.18) (layer F.Cu) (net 6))
 (segment (start 121.43 93.236) (end 120.414 94.252) (width 0.18) (layer F.Cu) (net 6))
 (segment (start 120.414 94.252) (end 120.414 101.11) (width 0.18) (layer F.Cu) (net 6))
 (segment (start 190.23 70.76) (end 142.89 70.76) (width 0.18) (layer F.Cu) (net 4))
 (segment (start 142.89 70.76) (end 120.414 93.236) (width 0.18) (layer F.Cu) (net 4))
 (segment (start 120.414 93.236) (end 119.398 94.252) (width 0.18) (layer F.Cu) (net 4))
 (segment (start 119.398 94.252) (end 119.398 101.872) (width 0.18) (layer F.Cu) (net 4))
 (segment (start 189.027919 93.62) (end 187.627919 92.22) (width 0.18) (layer F.Cu) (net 22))
 (segment (start 190.23 93.62) (end 189.027919 93.62) (width 0.18) (layer F.Cu) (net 22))
 (segment (start 187.627919 92.22) (end 150.386 92.22) (width 0.18) (layer F.Cu) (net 22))
 (segment (start 150.386 92.22) (end 149.37 93.236) (width 0.18) (layer F.Cu) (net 22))
 (segment (start 149.37 93.236) (end 149.37 98.57) (width 0.18) (layer F.Cu) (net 22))
 (segment (start 189.027919 91.08) (end 188.897919 90.95) (width 0.18) (layer F.Cu) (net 20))
 (segment (start 190.23 91.08) (end 189.027919 91.08) (width 0.18) (layer F.Cu) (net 20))
 (segment (start 188.897919 90.95) (end 151.656 90.95) (width 0.18) (layer F.Cu) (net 20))
 (segment (start 151.656 90.95) (end 150.64 90.95) (width 0.18) (layer F.Cu) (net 20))
 (segment (start 150.64 90.95) (end 148.354 93.236) (width 0.18) (layer F.Cu) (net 20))
 (segment (start 148.354 93.236) (end 148.354 99.332) (width 0.18) (layer F.Cu) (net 20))
 (segment (start 190.23 88.54) (end 152.034 88.54) (width 0.18) (layer F.Cu) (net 18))
 (segment (start 152.034 88.54) (end 147.338 93.236) (width 0.18) (layer F.Cu) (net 18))
 (segment (start 147.338 93.236) (end 147.338 100.094) (width 0.18) (layer F.Cu) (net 18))
 (segment (start 189.027919 86) (end 188.897919 85.87) (width 0.18) (layer F.Cu) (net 16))
 (segment (start 190.23 86) (end 189.027919 86) (width 0.18) (layer F.Cu) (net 16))
 (segment (start 188.897919 85.87) (end 155.212 85.87) (width 0.18) (layer F.Cu) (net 16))
 (segment (start 155.212 85.87) (end 153.688 85.87) (width 0.18) (layer F.Cu) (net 16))
 (segment (start 153.688 85.87) (end 146.322 93.236) (width 0.18) (layer F.Cu) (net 16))
 (segment (start 146.322 93.236) (end 146.322 100.856) (width 0.18) (layer F.Cu) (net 16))
 (segment (start 190.23 83.46) (end 155.082 83.46) (width 0.18) (layer F.Cu) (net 14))
 (segment (start 155.082 83.46) (end 145.306 93.236) (width 0.18) (layer F.Cu) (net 14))
 (segment (start 145.306 93.236) (end 145.306 101.618) (width 0.18) (layer F.Cu) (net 14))
 (segment (start 112 73.975) (end 112 71.38) (width 0.18) (layer F.Cu) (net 1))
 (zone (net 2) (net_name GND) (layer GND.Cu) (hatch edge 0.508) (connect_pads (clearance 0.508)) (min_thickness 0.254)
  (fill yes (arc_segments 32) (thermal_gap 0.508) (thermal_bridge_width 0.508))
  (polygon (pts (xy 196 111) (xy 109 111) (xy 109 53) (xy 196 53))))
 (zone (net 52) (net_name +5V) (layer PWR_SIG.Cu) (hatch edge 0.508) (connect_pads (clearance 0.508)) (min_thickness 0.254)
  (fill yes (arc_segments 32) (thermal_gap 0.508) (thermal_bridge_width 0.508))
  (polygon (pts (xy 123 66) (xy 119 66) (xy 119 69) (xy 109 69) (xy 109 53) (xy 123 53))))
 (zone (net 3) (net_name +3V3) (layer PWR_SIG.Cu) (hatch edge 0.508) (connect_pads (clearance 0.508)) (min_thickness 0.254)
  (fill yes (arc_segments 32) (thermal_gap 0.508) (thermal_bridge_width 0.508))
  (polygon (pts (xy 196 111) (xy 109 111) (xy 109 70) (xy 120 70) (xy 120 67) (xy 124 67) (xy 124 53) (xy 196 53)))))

